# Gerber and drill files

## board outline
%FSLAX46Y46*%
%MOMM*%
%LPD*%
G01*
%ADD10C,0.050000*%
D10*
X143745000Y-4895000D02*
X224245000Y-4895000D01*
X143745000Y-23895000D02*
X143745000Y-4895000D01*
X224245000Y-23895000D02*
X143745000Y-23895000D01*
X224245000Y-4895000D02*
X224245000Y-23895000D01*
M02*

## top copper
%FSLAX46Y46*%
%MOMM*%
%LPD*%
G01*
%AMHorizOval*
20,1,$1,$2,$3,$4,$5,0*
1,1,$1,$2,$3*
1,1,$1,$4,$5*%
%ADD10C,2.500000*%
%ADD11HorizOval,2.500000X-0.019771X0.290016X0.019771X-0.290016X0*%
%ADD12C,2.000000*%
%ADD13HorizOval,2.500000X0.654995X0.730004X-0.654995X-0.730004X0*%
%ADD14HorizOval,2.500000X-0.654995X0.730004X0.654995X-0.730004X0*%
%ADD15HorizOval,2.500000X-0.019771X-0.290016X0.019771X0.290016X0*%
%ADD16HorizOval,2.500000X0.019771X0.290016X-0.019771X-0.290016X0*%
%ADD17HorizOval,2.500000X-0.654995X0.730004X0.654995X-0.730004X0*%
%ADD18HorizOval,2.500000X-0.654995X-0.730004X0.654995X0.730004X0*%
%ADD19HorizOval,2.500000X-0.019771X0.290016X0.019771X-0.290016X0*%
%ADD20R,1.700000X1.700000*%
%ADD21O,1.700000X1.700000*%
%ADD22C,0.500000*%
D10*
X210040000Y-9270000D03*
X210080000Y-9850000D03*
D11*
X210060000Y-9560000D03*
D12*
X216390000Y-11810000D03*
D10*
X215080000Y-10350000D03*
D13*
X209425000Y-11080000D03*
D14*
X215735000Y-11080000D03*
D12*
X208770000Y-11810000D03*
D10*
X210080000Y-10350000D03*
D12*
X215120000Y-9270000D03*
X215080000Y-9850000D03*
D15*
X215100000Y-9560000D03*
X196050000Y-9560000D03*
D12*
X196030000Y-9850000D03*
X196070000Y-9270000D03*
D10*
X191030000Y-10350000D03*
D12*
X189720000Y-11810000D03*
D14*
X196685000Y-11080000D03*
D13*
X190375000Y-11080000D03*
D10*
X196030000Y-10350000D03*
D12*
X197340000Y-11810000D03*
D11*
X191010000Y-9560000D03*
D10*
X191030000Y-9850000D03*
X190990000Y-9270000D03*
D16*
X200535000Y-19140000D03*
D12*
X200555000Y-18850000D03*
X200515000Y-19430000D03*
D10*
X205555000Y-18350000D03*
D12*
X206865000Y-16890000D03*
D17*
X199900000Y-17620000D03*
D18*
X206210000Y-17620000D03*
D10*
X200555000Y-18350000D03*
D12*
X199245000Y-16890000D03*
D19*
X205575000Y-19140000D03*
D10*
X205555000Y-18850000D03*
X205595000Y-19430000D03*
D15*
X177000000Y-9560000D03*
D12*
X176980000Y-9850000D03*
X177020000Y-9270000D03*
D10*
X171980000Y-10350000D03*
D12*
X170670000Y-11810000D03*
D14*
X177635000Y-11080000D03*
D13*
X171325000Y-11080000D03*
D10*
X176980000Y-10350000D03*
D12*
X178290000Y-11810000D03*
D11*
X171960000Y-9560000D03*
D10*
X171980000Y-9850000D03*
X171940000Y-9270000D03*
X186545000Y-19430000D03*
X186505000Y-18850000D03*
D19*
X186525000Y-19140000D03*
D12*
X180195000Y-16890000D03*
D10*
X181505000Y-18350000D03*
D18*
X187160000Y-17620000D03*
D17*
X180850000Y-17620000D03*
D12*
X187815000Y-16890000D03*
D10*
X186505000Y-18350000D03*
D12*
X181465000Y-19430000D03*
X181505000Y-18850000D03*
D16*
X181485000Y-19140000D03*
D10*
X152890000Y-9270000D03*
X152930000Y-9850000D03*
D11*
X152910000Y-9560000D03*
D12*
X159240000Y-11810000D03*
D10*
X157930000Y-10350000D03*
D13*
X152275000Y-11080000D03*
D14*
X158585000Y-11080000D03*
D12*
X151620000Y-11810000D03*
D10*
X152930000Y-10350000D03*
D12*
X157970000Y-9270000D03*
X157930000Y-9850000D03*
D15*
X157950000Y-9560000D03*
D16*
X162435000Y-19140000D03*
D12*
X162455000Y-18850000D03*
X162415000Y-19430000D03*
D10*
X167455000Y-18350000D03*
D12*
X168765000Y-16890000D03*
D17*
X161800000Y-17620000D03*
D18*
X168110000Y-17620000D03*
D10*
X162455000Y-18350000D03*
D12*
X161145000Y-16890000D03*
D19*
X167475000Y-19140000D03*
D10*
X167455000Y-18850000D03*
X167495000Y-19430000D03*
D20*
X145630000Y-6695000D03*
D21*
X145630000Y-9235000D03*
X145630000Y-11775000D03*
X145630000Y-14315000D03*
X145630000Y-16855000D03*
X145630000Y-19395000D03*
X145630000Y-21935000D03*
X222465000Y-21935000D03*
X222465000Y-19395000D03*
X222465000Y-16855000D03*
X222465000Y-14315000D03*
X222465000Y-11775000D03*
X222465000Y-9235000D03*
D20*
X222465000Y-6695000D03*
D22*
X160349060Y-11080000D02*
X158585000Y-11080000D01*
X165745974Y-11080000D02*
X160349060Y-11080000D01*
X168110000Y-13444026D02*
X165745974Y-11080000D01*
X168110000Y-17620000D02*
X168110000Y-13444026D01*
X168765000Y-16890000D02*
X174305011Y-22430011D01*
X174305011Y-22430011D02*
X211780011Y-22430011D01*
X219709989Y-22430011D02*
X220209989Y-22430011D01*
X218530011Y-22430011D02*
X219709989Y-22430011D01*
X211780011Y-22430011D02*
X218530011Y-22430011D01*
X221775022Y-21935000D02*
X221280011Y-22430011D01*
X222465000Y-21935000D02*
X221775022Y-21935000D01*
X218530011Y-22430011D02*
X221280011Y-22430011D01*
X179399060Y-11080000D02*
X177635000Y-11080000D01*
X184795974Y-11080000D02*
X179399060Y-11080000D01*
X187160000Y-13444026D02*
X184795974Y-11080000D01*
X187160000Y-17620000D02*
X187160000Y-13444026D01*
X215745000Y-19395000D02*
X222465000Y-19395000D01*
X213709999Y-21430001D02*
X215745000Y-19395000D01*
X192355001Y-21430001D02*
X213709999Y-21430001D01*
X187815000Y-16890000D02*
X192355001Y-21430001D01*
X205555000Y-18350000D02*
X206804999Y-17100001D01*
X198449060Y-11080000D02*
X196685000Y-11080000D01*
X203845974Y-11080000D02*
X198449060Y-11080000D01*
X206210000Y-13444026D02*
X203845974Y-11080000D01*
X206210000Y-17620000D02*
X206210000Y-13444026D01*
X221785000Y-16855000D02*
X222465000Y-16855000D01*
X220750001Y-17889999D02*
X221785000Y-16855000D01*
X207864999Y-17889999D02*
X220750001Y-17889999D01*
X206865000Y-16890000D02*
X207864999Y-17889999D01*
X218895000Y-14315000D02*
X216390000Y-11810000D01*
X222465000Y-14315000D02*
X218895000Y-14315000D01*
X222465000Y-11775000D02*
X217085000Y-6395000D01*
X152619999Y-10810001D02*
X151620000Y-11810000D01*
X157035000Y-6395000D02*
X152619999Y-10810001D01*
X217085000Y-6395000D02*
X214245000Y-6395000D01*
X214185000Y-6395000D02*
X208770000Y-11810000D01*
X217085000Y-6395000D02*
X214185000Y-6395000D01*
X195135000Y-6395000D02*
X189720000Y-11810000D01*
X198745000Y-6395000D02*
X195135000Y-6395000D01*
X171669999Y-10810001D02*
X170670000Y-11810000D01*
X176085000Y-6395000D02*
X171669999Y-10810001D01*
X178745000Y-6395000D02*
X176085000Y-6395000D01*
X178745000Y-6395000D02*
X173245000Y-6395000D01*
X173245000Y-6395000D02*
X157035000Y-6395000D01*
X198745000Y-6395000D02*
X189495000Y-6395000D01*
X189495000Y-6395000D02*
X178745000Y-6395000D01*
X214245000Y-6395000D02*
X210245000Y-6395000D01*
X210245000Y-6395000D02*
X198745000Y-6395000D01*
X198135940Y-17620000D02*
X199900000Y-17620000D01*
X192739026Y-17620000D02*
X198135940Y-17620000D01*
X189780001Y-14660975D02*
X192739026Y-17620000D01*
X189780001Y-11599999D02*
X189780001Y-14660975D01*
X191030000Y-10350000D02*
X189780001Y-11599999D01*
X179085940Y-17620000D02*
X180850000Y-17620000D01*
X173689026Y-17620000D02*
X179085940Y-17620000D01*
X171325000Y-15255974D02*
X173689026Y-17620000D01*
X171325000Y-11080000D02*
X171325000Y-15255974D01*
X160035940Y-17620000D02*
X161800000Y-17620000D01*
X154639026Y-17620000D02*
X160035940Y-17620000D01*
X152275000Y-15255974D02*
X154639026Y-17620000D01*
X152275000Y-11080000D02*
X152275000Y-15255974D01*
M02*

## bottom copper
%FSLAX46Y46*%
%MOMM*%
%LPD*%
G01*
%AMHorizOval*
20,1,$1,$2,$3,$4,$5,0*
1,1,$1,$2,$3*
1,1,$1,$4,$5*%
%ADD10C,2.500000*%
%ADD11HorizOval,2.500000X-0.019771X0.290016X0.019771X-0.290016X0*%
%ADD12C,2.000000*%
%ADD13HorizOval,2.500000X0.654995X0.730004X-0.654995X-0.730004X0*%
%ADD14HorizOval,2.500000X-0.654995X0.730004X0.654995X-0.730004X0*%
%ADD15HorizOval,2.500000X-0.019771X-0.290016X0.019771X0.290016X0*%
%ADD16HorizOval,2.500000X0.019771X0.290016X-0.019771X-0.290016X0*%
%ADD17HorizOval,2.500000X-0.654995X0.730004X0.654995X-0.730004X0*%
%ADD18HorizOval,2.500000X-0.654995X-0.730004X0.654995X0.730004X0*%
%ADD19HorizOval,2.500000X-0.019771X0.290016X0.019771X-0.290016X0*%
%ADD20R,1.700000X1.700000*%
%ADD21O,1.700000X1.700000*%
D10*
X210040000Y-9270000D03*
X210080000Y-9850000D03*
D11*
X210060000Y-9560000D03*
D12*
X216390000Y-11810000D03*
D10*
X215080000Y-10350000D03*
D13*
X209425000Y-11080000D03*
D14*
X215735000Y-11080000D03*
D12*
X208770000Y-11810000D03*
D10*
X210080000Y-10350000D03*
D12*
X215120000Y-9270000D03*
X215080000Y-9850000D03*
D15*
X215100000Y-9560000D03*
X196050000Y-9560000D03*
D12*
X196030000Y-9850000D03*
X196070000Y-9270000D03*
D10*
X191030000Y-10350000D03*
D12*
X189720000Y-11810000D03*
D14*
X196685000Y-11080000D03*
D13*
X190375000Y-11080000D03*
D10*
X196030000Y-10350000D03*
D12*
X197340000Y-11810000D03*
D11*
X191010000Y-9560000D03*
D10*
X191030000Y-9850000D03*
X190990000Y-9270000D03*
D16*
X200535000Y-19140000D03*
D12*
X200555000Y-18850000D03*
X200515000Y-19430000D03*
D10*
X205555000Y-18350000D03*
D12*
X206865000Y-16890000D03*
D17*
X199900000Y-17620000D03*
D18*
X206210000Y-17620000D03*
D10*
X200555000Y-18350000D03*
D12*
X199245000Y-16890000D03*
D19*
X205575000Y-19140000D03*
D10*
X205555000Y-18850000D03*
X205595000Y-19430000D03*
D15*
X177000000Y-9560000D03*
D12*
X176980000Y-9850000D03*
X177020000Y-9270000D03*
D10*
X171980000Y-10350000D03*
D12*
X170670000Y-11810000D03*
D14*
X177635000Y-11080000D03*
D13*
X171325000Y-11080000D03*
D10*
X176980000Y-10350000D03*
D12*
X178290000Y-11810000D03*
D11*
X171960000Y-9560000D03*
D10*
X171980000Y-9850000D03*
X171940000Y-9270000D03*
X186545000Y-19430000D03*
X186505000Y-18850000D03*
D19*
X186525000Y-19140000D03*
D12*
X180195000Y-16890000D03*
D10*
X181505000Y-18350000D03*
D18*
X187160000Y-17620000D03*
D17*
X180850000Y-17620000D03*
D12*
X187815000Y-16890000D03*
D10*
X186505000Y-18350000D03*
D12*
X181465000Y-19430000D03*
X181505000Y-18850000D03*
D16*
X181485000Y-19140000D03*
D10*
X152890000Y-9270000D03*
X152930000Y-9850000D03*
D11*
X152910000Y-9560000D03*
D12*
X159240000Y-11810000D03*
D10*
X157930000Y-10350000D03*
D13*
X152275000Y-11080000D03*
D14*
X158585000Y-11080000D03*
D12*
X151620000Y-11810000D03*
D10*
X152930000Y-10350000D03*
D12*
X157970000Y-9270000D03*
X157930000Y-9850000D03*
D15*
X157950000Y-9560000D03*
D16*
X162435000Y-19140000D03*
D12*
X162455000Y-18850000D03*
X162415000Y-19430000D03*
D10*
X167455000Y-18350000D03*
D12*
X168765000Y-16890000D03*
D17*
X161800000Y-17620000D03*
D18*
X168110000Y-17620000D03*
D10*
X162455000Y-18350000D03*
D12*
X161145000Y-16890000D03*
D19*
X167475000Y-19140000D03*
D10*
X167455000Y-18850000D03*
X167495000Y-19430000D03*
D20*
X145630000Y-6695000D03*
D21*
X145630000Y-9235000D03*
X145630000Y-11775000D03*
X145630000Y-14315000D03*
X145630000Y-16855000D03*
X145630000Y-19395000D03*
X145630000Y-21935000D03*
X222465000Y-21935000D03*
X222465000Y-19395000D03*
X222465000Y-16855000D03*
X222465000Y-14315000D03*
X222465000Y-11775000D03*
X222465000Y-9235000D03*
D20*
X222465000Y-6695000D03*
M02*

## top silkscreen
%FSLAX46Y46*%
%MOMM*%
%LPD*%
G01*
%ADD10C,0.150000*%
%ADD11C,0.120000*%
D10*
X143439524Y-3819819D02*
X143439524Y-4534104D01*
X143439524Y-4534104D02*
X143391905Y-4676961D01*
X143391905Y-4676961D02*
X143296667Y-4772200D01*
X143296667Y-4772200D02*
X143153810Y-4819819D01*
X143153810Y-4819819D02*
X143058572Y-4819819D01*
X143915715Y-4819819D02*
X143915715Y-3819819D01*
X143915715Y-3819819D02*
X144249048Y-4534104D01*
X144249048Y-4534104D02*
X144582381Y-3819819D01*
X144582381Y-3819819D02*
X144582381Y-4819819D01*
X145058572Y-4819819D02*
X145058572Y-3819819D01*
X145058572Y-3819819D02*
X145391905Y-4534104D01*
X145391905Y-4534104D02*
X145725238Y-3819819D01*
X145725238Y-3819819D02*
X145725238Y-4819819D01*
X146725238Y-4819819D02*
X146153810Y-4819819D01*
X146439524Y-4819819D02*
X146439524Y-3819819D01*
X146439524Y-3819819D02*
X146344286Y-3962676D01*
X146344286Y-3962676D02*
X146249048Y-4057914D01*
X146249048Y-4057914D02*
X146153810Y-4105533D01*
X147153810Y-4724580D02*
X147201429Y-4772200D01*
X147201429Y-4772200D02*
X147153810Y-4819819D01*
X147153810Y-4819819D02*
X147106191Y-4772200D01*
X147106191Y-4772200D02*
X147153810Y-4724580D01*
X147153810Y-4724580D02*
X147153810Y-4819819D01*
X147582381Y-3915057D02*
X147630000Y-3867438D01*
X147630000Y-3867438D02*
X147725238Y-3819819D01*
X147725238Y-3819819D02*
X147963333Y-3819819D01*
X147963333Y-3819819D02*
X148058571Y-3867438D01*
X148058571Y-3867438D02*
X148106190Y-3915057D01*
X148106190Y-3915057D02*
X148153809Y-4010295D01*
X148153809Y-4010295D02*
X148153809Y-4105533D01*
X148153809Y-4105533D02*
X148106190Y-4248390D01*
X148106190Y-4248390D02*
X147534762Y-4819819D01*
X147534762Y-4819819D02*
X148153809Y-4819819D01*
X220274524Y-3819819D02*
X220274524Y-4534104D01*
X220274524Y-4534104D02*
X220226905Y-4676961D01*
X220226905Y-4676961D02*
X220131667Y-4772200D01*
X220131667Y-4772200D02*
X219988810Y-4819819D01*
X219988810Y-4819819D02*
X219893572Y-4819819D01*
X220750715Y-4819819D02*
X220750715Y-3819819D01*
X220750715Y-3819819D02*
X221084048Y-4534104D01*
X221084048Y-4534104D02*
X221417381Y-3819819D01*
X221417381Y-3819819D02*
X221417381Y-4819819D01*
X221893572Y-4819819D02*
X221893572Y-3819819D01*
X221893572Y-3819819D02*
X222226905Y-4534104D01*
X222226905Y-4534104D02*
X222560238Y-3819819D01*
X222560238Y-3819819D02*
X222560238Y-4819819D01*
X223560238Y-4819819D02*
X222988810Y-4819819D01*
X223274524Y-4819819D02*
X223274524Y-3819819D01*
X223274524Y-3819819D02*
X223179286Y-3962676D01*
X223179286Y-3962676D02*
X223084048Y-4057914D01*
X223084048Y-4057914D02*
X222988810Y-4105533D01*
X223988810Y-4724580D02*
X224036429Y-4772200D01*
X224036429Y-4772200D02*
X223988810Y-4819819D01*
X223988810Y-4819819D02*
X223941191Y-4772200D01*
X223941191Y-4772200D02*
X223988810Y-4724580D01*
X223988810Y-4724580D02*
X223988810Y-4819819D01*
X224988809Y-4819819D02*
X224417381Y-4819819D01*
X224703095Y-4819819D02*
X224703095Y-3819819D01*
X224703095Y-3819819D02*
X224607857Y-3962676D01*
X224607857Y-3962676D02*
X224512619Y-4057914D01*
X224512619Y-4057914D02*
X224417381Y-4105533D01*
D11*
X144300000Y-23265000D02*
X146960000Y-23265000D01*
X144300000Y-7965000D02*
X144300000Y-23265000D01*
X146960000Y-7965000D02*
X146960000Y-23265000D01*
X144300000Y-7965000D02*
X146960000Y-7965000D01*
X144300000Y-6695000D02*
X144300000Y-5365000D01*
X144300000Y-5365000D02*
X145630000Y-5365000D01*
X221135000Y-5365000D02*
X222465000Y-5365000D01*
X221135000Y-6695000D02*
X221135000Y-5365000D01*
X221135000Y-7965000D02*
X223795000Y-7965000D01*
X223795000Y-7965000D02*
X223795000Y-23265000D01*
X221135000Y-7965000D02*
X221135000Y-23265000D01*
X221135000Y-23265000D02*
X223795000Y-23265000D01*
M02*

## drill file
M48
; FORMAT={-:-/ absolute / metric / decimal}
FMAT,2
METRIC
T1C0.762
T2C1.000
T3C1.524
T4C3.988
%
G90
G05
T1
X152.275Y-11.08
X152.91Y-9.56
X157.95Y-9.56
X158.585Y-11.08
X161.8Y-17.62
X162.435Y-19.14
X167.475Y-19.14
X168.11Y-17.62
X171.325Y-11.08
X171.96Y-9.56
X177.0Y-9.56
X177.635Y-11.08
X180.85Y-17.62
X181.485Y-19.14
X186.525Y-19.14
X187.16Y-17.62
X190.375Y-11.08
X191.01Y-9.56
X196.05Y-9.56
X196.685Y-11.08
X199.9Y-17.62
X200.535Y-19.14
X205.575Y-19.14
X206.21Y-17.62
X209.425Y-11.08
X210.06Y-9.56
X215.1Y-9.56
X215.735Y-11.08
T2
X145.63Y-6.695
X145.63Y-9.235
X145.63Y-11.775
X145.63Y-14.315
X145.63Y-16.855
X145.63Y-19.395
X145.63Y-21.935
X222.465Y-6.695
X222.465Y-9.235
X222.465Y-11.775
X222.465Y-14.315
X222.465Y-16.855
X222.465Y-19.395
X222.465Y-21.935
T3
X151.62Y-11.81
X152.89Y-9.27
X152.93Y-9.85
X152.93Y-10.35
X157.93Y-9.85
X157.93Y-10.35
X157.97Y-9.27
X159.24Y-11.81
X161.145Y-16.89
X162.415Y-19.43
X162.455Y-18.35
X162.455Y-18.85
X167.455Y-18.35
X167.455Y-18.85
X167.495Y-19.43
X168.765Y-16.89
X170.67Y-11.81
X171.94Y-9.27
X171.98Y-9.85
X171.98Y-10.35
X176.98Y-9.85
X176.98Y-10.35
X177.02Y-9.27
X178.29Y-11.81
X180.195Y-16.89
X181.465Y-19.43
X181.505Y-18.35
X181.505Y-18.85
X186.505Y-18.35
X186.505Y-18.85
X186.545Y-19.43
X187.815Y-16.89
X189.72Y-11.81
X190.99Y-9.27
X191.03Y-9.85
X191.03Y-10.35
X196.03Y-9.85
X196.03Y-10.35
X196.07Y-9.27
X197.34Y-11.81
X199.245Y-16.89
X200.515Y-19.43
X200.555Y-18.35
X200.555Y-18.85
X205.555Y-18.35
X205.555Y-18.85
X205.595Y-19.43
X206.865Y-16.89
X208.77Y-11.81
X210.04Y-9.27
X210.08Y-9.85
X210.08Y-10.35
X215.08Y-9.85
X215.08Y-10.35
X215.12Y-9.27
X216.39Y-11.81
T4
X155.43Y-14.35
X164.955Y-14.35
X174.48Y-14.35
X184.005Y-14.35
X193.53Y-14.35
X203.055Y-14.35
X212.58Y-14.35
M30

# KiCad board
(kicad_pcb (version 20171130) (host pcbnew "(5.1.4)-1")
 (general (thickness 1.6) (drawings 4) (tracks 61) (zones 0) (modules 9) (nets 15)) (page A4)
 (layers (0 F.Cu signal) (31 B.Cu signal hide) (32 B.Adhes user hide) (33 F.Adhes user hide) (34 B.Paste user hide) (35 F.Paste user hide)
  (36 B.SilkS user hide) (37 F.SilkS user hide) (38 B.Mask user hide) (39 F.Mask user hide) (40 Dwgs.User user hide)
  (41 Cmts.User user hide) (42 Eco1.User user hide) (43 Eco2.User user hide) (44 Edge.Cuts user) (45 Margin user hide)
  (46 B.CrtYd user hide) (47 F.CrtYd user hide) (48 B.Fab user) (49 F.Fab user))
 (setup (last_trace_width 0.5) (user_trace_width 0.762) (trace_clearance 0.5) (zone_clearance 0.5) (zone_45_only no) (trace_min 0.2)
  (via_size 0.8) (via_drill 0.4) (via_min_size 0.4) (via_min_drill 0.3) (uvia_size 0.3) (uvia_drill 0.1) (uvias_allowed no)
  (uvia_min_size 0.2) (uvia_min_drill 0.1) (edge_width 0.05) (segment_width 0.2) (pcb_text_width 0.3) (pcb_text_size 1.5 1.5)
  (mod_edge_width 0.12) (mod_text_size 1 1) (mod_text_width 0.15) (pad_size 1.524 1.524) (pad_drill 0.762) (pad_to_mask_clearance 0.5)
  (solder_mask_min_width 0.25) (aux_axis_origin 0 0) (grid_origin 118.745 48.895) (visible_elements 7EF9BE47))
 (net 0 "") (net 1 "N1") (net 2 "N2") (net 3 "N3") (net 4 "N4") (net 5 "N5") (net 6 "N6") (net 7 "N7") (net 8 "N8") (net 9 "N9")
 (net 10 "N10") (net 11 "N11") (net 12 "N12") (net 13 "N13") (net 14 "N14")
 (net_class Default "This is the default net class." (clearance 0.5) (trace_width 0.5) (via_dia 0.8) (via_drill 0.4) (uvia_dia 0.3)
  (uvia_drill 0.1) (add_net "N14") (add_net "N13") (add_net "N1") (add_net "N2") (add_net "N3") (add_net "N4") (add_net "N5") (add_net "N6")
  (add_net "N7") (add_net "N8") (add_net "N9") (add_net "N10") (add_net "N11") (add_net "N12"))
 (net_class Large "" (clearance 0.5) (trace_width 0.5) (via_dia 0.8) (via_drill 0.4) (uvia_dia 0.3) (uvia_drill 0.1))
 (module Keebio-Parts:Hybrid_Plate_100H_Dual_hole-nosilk (layer F.Cu) (at 212.58 14.35)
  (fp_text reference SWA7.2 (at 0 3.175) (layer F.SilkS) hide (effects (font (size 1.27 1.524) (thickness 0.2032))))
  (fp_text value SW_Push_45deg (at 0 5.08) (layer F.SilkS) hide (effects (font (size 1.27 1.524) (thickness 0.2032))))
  (pad 1 thru_hole circle (at -2.54 -5.08 330.9) (size 2.5 2.5) (drill 1.524) (layers *.Cu F.Mask) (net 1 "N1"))
  (pad 1 thru_hole circle (at -2.5 -4.5 330.9) (size 2.5 2.5) (drill 1.524) (layers *.Cu F.Mask) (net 1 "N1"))
  (pad 1 thru_hole oval (at -2.52 -4.79 3.9) (size 2.5 3.081378) (drill 0.762) (layers *.Cu F.Mask) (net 1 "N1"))
  (pad 2 thru_hole circle (at 3.81 -2.54 330.9) (size 2 2) (drill 1.524) (layers *.Cu F.Mask) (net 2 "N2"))
  (pad 2 thru_hole circle (at 2.5 -4) (size 2.5 2.5) (drill 1.524) (layers *.Cu *.Mask) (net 2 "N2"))
  (pad 1 thru_hole oval (at -3.155 -3.27 138.1) (size 2.5 4.461556) (drill 0.762) (layers *.Cu B.Mask) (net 1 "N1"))
  (pad 2 thru_hole oval (at 3.155 -3.27 221.9) (size 2.5 4.461556) (drill 0.762) (layers *.Cu F.Mask) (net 2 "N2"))
  (pad 1 thru_hole circle (at -3.81 -2.54 330.9) (size 2 2) (drill 1.524) (layers *.Cu B.Mask) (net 1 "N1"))
  (pad HOLE np_thru_hole circle (at 0 0) (size 3.9878 3.9878) (drill 3.9878) (layers *.Cu *.Mask))
  (pad 1 thru_hole circle (at -2.5 -4 330.9) (size 2.5 2.5) (drill 1.524) (layers *.Cu *.Mask) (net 1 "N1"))
  (pad 2 thru_hole circle (at 2.54 -5.08 330.9) (size 2 2) (drill 1.524) (layers *.Cu B.Mask) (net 2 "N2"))
  (pad 2 thru_hole circle (at 2.5 -4.5 330.9) (size 2 2) (drill 1.524) (layers *.Cu B.Mask) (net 2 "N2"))
  (pad 2 thru_hole oval (at 2.52 -4.79 356.1) (size 2.5 3.081378) (drill 0.762) (layers *.Cu B.Mask) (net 2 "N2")))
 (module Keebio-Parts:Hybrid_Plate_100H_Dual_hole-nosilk (layer F.Cu) (at 193.53 14.35)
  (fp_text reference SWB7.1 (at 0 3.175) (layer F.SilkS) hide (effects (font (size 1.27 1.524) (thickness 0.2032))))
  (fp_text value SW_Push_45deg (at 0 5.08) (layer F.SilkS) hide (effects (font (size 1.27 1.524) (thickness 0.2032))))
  (pad 2 thru_hole oval (at 2.52 -4.79 356.1) (size 2.5 3.081378) (drill 0.762) (layers *.Cu B.Mask) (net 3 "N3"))
  (pad 2 thru_hole circle (at 2.5 -4.5 330.9) (size 2 2) (drill 1.524) (layers *.Cu B.Mask) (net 3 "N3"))
  (pad 2 thru_hole circle (at 2.54 -5.08 330.9) (size 2 2) (drill 1.524) (layers *.Cu B.Mask) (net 3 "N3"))
  (pad 1 thru_hole circle (at -2.5 -4 330.9) (size 2.5 2.5) (drill 1.524) (layers *.Cu *.Mask) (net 1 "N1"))
  (pad HOLE np_thru_hole circle (at 0 0) (size 3.9878 3.9878) (drill 3.9878) (layers *.Cu *.Mask))
  (pad 1 thru_hole circle (at -3.81 -2.54 330.9) (size 2 2) (drill 1.524) (layers *.Cu B.Mask) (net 1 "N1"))
  (pad 2 thru_hole oval (at 3.155 -3.27 221.9) (size 2.5 4.461556) (drill 0.762) (layers *.Cu F.Mask) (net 3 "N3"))
  (pad 1 thru_hole oval (at -3.155 -3.27 138.1) (size 2.5 4.461556) (drill 0.762) (layers *.Cu B.Mask) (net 1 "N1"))
  (pad 2 thru_hole circle (at 2.5 -4) (size 2.5 2.5) (drill 1.524) (layers *.Cu *.Mask) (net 3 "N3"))
  (pad 2 thru_hole circle (at 3.81 -2.54 330.9) (size 2 2) (drill 1.524) (layers *.Cu F.Mask) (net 3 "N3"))
  (pad 1 thru_hole oval (at -2.52 -4.79 3.9) (size 2.5 3.081378) (drill 0.762) (layers *.Cu F.Mask) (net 1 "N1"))
  (pad 1 thru_hole circle (at -2.5 -4.5 330.9) (size 2.5 2.5) (drill 1.524) (layers *.Cu F.Mask) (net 1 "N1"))
  (pad 1 thru_hole circle (at -2.54 -5.08 330.9) (size 2.5 2.5) (drill 1.524) (layers *.Cu F.Mask) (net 1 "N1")))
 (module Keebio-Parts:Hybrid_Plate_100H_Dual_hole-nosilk (layer F.Cu) (at 203.055 14.35 180)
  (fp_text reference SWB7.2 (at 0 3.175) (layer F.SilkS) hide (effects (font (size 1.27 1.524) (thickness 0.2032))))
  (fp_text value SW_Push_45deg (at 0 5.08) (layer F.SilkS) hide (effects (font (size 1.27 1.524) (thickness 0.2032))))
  (pad 2 thru_hole oval (at 2.52 -4.79 176.1) (size 2.5 3.081378) (drill 0.762) (layers *.Cu B.Mask) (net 1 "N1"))
  (pad 2 thru_hole circle (at 2.5 -4.5 150.9) (size 2 2) (drill 1.524) (layers *.Cu B.Mask) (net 1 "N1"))
  (pad 2 thru_hole circle (at 2.54 -5.08 150.9) (size 2 2) (drill 1.524) (layers *.Cu B.Mask) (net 1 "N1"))
  (pad 1 thru_hole circle (at -2.5 -4 150.9) (size 2.5 2.5) (drill 1.524) (layers *.Cu *.Mask) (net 3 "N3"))
  (pad HOLE np_thru_hole circle (at 0 0 180) (size 3.9878 3.9878) (drill 3.9878) (layers *.Cu *.Mask))
  (pad 1 thru_hole circle (at -3.81 -2.54 150.9) (size 2 2) (drill 1.524) (layers *.Cu B.Mask) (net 3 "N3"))
  (pad 2 thru_hole oval (at 3.155 -3.27 41.9) (size 2.5 4.461556) (drill 0.762) (layers *.Cu F.Mask) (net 1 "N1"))
  (pad 1 thru_hole oval (at -3.155 -3.27 318.1) (size 2.5 4.461556) (drill 0.762) (layers *.Cu B.Mask) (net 3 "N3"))
  (pad 2 thru_hole circle (at 2.5 -4 180) (size 2.5 2.5) (drill 1.524) (layers *.Cu *.Mask) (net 1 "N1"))
  (pad 2 thru_hole circle (at 3.81 -2.54 150.9) (size 2 2) (drill 1.524) (layers *.Cu F.Mask) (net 1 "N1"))
  (pad 1 thru_hole oval (at -2.52 -4.79 183.9) (size 2.5 3.081378) (drill 0.762) (layers *.Cu F.Mask) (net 3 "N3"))
  (pad 1 thru_hole circle (at -2.5 -4.5 150.9) (size 2.5 2.5) (drill 1.524) (layers *.Cu F.Mask) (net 3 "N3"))
  (pad 1 thru_hole circle (at -2.54 -5.08 150.9) (size 2.5 2.5) (drill 1.524) (layers *.Cu F.Mask) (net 3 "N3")))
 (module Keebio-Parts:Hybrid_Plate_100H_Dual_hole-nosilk (layer F.Cu) (at 174.48 14.35)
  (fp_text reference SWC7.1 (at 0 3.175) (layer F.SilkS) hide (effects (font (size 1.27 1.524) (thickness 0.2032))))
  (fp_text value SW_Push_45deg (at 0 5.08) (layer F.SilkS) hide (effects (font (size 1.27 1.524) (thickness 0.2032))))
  (pad 2 thru_hole oval (at 2.52 -4.79 356.1) (size 2.5 3.081378) (drill 0.762) (layers *.Cu B.Mask) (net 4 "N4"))
  (pad 2 thru_hole circle (at 2.5 -4.5 330.9) (size 2 2) (drill 1.524) (layers *.Cu B.Mask) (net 4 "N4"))
  (pad 2 thru_hole circle (at 2.54 -5.08 330.9) (size 2 2) (drill 1.524) (layers *.Cu B.Mask) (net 4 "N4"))
  (pad 1 thru_hole circle (at -2.5 -4 330.9) (size 2.5 2.5) (drill 1.524) (layers *.Cu *.Mask) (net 1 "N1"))
  (pad HOLE np_thru_hole circle (at 0 0) (size 3.9878 3.9878) (drill 3.9878) (layers *.Cu *.Mask))
  (pad 1 thru_hole circle (at -3.81 -2.54 330.9) (size 2 2) (drill 1.524) (layers *.Cu B.Mask) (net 1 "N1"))
  (pad 2 thru_hole oval (at 3.155 -3.27 221.9) (size 2.5 4.461556) (drill 0.762) (layers *.Cu F.Mask) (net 4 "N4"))
  (pad 1 thru_hole oval (at -3.155 -3.27 138.1) (size 2.5 4.461556) (drill 0.762) (layers *.Cu B.Mask) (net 1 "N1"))
  (pad 2 thru_hole circle (at 2.5 -4) (size 2.5 2.5) (drill 1.524) (layers *.Cu *.Mask) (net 4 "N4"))
  (pad 2 thru_hole circle (at 3.81 -2.54 330.9) (size 2 2) (drill 1.524) (layers *.Cu F.Mask) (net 4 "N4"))
  (pad 1 thru_hole oval (at -2.52 -4.79 3.9) (size 2.5 3.081378) (drill 0.762) (layers *.Cu F.Mask) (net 1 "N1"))
  (pad 1 thru_hole circle (at -2.5 -4.5 330.9) (size 2.5 2.5) (drill 1.524) (layers *.Cu F.Mask) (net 1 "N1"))
  (pad 1 thru_hole circle (at -2.54 -5.08 330.9) (size 2.5 2.5) (drill 1.524) (layers *.Cu F.Mask) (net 1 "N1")))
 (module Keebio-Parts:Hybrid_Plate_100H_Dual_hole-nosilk (layer F.Cu) (at 184.005 14.35 180)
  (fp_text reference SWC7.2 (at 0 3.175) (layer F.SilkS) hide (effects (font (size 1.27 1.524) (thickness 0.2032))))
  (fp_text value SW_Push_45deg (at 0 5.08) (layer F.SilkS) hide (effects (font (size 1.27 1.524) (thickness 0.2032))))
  (pad 1 thru_hole circle (at -2.54 -5.08 150.9) (size 2.5 2.5) (drill 1.524) (layers *.Cu F.Mask) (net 4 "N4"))
  (pad 1 thru_hole circle (at -2.5 -4.5 150.9) (size 2.5 2.5) (drill 1.524) (layers *.Cu F.Mask) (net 4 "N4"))
  (pad 1 thru_hole oval (at -2.52 -4.79 183.9) (size 2.5 3.081378) (drill 0.762) (layers *.Cu F.Mask) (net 4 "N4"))
  (pad 2 thru_hole circle (at 3.81 -2.54 150.9) (size 2 2) (drill 1.524) (layers *.Cu F.Mask) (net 1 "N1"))
  (pad 2 thru_hole circle (at 2.5 -4 180) (size 2.5 2.5) (drill 1.524) (layers *.Cu *.Mask) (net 1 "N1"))
  (pad 1 thru_hole oval (at -3.155 -3.27 318.1) (size 2.5 4.461556) (drill 0.762) (layers *.Cu B.Mask) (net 4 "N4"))
  (pad 2 thru_hole oval (at 3.155 -3.27 41.9) (size 2.5 4.461556) (drill 0.762) (layers *.Cu F.Mask) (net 1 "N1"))
  (pad 1 thru_hole circle (at -3.81 -2.54 150.9) (size 2 2) (drill 1.524) (layers *.Cu B.Mask) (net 4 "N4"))
  (pad HOLE np_thru_hole circle (at 0 0 180) (size 3.9878 3.9878) (drill 3.9878) (layers *.Cu *.Mask))
  (pad 1 thru_hole circle (at -2.5 -4 150.9) (size 2.5 2.5) (drill 1.524) (layers *.Cu *.Mask) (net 4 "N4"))
  (pad 2 thru_hole circle (at 2.54 -5.08 150.9) (size 2 2) (drill 1.524) (layers *.Cu B.Mask) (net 1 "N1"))
  (pad 2 thru_hole circle (at 2.5 -4.5 150.9) (size 2 2) (drill 1.524) (layers *.Cu B.Mask) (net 1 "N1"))
  (pad 2 thru_hole oval (at 2.52 -4.79 176.1) (size 2.5 3.081378) (drill 0.762) (layers *.Cu B.Mask) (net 1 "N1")))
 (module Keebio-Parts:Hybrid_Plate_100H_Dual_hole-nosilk (layer F.Cu) (at 155.43 14.35)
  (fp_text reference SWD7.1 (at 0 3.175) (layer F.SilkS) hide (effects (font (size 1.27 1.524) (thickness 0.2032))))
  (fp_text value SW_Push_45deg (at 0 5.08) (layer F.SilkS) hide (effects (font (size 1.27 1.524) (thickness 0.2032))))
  (pad 1 thru_hole circle (at -2.54 -5.08 330.9) (size 2.5 2.5) (drill 1.524) (layers *.Cu F.Mask) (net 1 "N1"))
  (pad 1 thru_hole circle (at -2.5 -4.5 330.9) (size 2.5 2.5) (drill 1.524) (layers *.Cu F.Mask) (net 1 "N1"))
  (pad 1 thru_hole oval (at -2.52 -4.79 3.9) (size 2.5 3.081378) (drill 0.762) (layers *.Cu F.Mask) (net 1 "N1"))
  (pad 2 thru_hole circle (at 3.81 -2.54 330.9) (size 2 2) (drill 1.524) (layers *.Cu F.Mask) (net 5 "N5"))
  (pad 2 thru_hole circle (at 2.5 -4) (size 2.5 2.5) (drill 1.524) (layers *.Cu *.Mask) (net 5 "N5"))
  (pad 1 thru_hole oval (at -3.155 -3.27 138.1) (size 2.5 4.461556) (drill 0.762) (layers *.Cu B.Mask) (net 1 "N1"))
  (pad 2 thru_hole oval (at 3.155 -3.27 221.9) (size 2.5 4.461556) (drill 0.762) (layers *.Cu F.Mask) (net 5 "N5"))
  (pad 1 thru_hole circle (at -3.81 -2.54 330.9) (size 2 2) (drill 1.524) (layers *.Cu B.Mask) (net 1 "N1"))
  (pad HOLE np_thru_hole circle (at 0 0) (size 3.9878 3.9878) (drill 3.9878) (layers *.Cu *.Mask))
  (pad 1 thru_hole circle (at -2.5 -4 330.9) (size 2.5 2.5) (drill 1.524) (layers *.Cu *.Mask) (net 1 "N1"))
  (pad 2 thru_hole circle (at 2.54 -5.08 330.9) (size 2 2) (drill 1.524) (layers *.Cu B.Mask) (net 5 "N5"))
  (pad 2 thru_hole circle (at 2.5 -4.5 330.9) (size 2 2) (drill 1.524) (layers *.Cu B.Mask) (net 5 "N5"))
  (pad 2 thru_hole oval (at 2.52 -4.79 356.1) (size 2.5 3.081378) (drill 0.762) (layers *.Cu B.Mask) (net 5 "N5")))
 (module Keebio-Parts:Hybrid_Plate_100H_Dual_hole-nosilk (layer F.Cu) (at 164.955 14.35 180)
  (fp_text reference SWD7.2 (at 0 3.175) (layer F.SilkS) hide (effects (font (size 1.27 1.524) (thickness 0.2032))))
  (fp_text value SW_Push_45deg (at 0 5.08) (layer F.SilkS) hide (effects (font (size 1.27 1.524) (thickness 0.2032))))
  (pad 2 thru_hole oval (at 2.52 -4.79 176.1) (size 2.5 3.081378) (drill 0.762) (layers *.Cu B.Mask) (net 1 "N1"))
  (pad 2 thru_hole circle (at 2.5 -4.5 150.9) (size 2 2) (drill 1.524) (layers *.Cu B.Mask) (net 1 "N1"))
  (pad 2 thru_hole circle (at 2.54 -5.08 150.9) (size 2 2) (drill 1.524) (layers *.Cu B.Mask) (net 1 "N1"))
  (pad 1 thru_hole circle (at -2.5 -4 150.9) (size 2.5 2.5) (drill 1.524) (layers *.Cu *.Mask) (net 5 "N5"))
  (pad HOLE np_thru_hole circle (at 0 0 180) (size 3.9878 3.9878) (drill 3.9878) (layers *.Cu *.Mask))
  (pad 1 thru_hole circle (at -3.81 -2.54 150.9) (size 2 2) (drill 1.524) (layers *.Cu B.Mask) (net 5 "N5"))
  (pad 2 thru_hole oval (at 3.155 -3.27 41.9) (size 2.5 4.461556) (drill 0.762) (layers *.Cu F.Mask) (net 1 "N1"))
  (pad 1 thru_hole oval (at -3.155 -3.27 318.1) (size 2.5 4.461556) (drill 0.762) (layers *.Cu B.Mask) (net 5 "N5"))
  (pad 2 thru_hole circle (at 2.5 -4 180) (size 2.5 2.5) (drill 1.524) (layers *.Cu *.Mask) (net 1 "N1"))
  (pad 2 thru_hole circle (at 3.81 -2.54 150.9) (size 2 2) (drill 1.524) (layers *.Cu F.Mask) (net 1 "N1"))
  (pad 1 thru_hole oval (at -2.52 -4.79 183.9) (size 2.5 3.081378) (drill 0.762) (layers *.Cu F.Mask) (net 5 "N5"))
  (pad 1 thru_hole circle (at -2.5 -4.5 150.9) (size 2.5 2.5) (drill 1.524) (layers *.Cu F.Mask) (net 5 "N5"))
  (pad 1 thru_hole circle (at -2.54 -5.08 150.9) (size 2.5 2.5) (drill 1.524) (layers *.Cu F.Mask) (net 5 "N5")))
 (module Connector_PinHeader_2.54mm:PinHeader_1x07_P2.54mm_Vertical (layer F.Cu) (at 145.63 6.695)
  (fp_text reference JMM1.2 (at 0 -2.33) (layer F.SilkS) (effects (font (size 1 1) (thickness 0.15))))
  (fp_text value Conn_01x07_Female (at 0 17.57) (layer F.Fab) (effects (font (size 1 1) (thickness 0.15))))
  (fp_line (start -1.33 16.57) (end 1.33 16.57) (layer F.SilkS) (width 0.12))
  (fp_line (start -1.33 1.27) (end -1.33 16.57) (layer F.SilkS) (width 0.12))
  (fp_line (start 1.33 1.27) (end 1.33 16.57) (layer F.SilkS) (width 0.12))
  (fp_line (start -1.33 1.27) (end 1.33 1.27) (layer F.SilkS) (width 0.12))
  (fp_line (start -1.33 0) (end -1.33 -1.33) (layer F.SilkS) (width 0.12))
  (fp_line (start -1.33 -1.33) (end 0 -1.33) (layer F.SilkS) (width 0.12))
  (pad 1 thru_hole rect (at 0 0) (size 1.7 1.7) (drill 1) (layers *.Cu *.Mask) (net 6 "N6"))
  (pad 2 thru_hole oval (at 0 2.54) (size 1.7 1.7) (drill 1) (layers *.Cu *.Mask) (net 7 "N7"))
  (pad 3 thru_hole oval (at 0 5.08) (size 1.7 1.7) (drill 1) (layers *.Cu *.Mask) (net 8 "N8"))
  (pad 4 thru_hole oval (at 0 7.62) (size 1.7 1.7) (drill 1) (layers *.Cu *.Mask) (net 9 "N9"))
  (pad 5 thru_hole oval (at 0 10.16) (size 1.7 1.7) (drill 1) (layers *.Cu *.Mask) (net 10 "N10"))
  (pad 6 thru_hole oval (at 0 12.7) (size 1.7 1.7) (drill 1) (layers *.Cu *.Mask) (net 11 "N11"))
  (pad 7 thru_hole oval (at 0 15.24) (size 1.7 1.7) (drill 1) (layers *.Cu *.Mask) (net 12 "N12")))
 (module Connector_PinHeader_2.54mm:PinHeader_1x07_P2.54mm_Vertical (layer F.Cu) (at 222.465 6.695)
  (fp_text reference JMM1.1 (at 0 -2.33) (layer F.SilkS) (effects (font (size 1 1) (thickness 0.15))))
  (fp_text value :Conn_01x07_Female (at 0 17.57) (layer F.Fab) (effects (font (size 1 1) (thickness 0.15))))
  (fp_line (start -1.33 -1.33) (end 0 -1.33) (layer F.SilkS) (width 0.12))
  (fp_line (start -1.33 0) (end -1.33 -1.33) (layer F.SilkS) (width 0.12))
  (fp_line (start -1.33 1.27) (end 1.33 1.27) (layer F.SilkS) (width 0.12))
  (fp_line (start 1.33 1.27) (end 1.33 16.57) (layer F.SilkS) (width 0.12))
  (fp_line (start -1.33 1.27) (end -1.33 16.57) (layer F.SilkS) (width 0.12))
  (fp_line (start -1.33 16.57) (end 1.33 16.57) (layer F.SilkS) (width 0.12))
  (pad 7 thru_hole oval (at 0 15.24) (size 1.7 1.7) (drill 1) (layers *.Cu *.Mask) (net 5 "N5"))
  (pad 6 thru_hole oval (at 0 12.7) (size 1.7 1.7) (drill 1) (layers *.Cu *.Mask) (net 4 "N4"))
  (pad 5 thru_hole oval (at 0 10.16) (size 1.7 1.7) (drill 1) (layers *.Cu *.Mask) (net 3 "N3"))
  (pad 4 thru_hole oval (at 0 7.62) (size 1.7 1.7) (drill 1) (layers *.Cu *.Mask) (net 2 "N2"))
  (pad 3 thru_hole oval (at 0 5.08) (size 1.7 1.7) (drill 1) (layers *.Cu *.Mask) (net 1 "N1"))
  (pad 2 thru_hole oval (at 0 2.54) (size 1.7 1.7) (drill 1) (layers *.Cu *.Mask) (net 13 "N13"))
  (pad 1 thru_hole rect (at 0 0) (size 1.7 1.7) (drill 1) (layers *.Cu *.Mask) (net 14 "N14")))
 (gr_line (start 143.745 4.895) (end 224.245 4.895) (layer Edge.Cuts) (width 0.05))
 (gr_line (start 143.745 23.895) (end 143.745 4.895) (layer Edge.Cuts) (width 0.05))
 (gr_line (start 224.245 23.895) (end 143.745 23.895) (layer Edge.Cuts) (width 0.05))
 (gr_line (start 224.245 4.895) (end 224.245 23.895) (layer Edge.Cuts) (width 0.05))
 (segment (start 160.34906 11.08) (end 158.585 11.08) (width 0.5) (layer F.Cu) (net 5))
 (segment (start 165.745974 11.08) (end 160.34906 11.08) (width 0.5) (layer F.Cu) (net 5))
 (segment (start 168.11 13.444026) (end 165.745974 11.08) (width 0.5) (layer F.Cu) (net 5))
 (segment (start 168.11 17.62) (end 168.11 13.444026) (width 0.5) (layer F.Cu) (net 5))
 (segment (start 168.765 16.89) (end 174.305011 22.430011) (width 0.5) (layer F.Cu) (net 5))
 (segment (start 174.305011 22.430011) (end 211.780011 22.430011) (width 0.5) (layer F.Cu) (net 5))
 (segment (start 219.709989 22.430011) (end 220.209989 22.430011) (width 0.5) (layer F.Cu) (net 5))
 (segment (start 218.530011 22.430011) (end 219.709989 22.430011) (width 0.5) (layer F.Cu) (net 5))
 (segment (start 211.780011 22.430011) (end 218.530011 22.430011) (width 0.5) (layer F.Cu) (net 5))
 (segment (start 221.775022 21.935) (end 221.280011 22.430011) (width 0.5) (layer F.Cu) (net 5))
 (segment (start 222.465 21.935) (end 221.775022 21.935) (width 0.5) (layer F.Cu) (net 5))
 (segment (start 218.530011 22.430011) (end 221.280011 22.430011) (width 0.5) (layer F.Cu) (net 5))
 (segment (start 179.39906 11.08) (end 177.635 11.08) (width 0.5) (layer F.Cu) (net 4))
 (segment (start 184.795974 11.08) (end 179.39906 11.08) (width 0.5) (layer F.Cu) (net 4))
 (segment (start 187.16 13.444026) (end 184.795974 11.08) (width 0.5) (layer F.Cu) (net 4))
 (segment (start 187.16 17.62) (end 187.16 13.444026) (width 0.5) (layer F.Cu) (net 4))
 (segment (start 215.745 19.395) (end 222.465 19.395) (width 0.5) (layer F.Cu) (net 4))
 (segment (start 213.709999 21.430001) (end 215.745 19.395) (width 0.5) (layer F.Cu) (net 4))
 (segment (start 192.355001 21.430001) (end 213.709999 21.430001) (width 0.5) (layer F.Cu) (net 4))
 (segment (start 187.815 16.89) (end 192.355001 21.430001) (width 0.5) (layer F.Cu) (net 4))
 (segment (start 205.555 18.35) (end 206.804999 17.100001) (width 0.5) (layer F.Cu) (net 3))
 (segment (start 198.44906 11.08) (end 196.685 11.08) (width 0.5) (layer F.Cu) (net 3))
 (segment (start 203.845974 11.08) (end 198.44906 11.08) (width 0.5) (layer F.Cu) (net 3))
 (segment (start 206.21 13.444026) (end 203.845974 11.08) (width 0.5) (layer F.Cu) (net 3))
 (segment (start 206.21 17.62) (end 206.21 13.444026) (width 0.5) (layer F.Cu) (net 3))
 (segment (start 221.785 16.855) (end 222.465 16.855) (width 0.5) (layer F.Cu) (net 3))
 (segment (start 220.750001 17.889999) (end 221.785 16.855) (width 0.5) (layer F.Cu) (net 3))
 (segment (start 207.864999 17.889999) (end 220.750001 17.889999) (width 0.5) (layer F.Cu) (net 3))
 (segment (start 206.865 16.89) (end 207.864999 17.889999) (width 0.5) (layer F.Cu) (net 3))
 (segment (start 218.895 14.315) (end 216.39 11.81) (width 0.5) (layer F.Cu) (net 2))
 (segment (start 222.465 14.315) (end 218.895 14.315) (width 0.5) (layer F.Cu) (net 2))
 (segment (start 222.465 11.775) (end 217.085 6.395) (width 0.5) (layer F.Cu) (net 1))
 (segment (start 152.619999 10.810001) (end 151.62 11.81) (width 0.5) (layer F.Cu) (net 1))
 (segment (start 157.035 6.395) (end 152.619999 10.810001) (width 0.5) (layer F.Cu) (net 1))
 (segment (start 217.085 6.395) (end 214.245 6.395) (width 0.5) (layer F.Cu) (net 1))
 (segment (start 214.185 6.395) (end 208.77 11.81) (width 0.5) (layer F.Cu) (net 1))
 (segment (start 217.085 6.395) (end 214.185 6.395) (width 0.5) (layer F.Cu) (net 1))
 (segment (start 195.135 6.395) (end 189.72 11.81) (width 0.5) (layer F.Cu) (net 1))
 (segment (start 198.745 6.395) (end 195.135 6.395) (width 0.5) (layer F.Cu) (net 1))
 (segment (start 171.669999 10.810001) (end 170.67 11.81) (width 0.5) (layer F.Cu) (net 1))
 (segment (start 176.085 6.395) (end 171.669999 10.810001) (width 0.5) (layer F.Cu) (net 1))
 (segment (start 178.745 6.395) (end 176.085 6.395) (width 0.5) (layer F.Cu) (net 1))
 (segment (start 178.745 6.395) (end 173.245 6.395) (width 0.5) (layer F.Cu) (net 1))
 (segment (start 173.245 6.395) (end 157.035 6.395) (width 0.5) (layer F.Cu) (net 1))
 (segment (start 198.745 6.395) (end 189.495 6.395) (width 0.5) (layer F.Cu) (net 1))
 (segment (start 189.495 6.395) (end 178.745 6.395) (width 0.5) (layer F.Cu) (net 1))
 (segment (start 214.245 6.395) (end 210.245 6.395) (width 0.5) (layer F.Cu) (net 1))
 (segment (start 210.245 6.395) (end 198.745 6.395) (width 0.5) (layer F.Cu) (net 1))
 (segment (start 198.13594 17.62) (end 199.9 17.62) (width 0.5) (layer F.Cu) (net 1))
 (segment (start 192.739026 17.62) (end 198.13594 17.62) (width 0.5) (layer F.Cu) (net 1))
 (segment (start 189.780001 14.660975) (end 192.739026 17.62) (width 0.5) (layer F.Cu) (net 1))
 (segment (start 189.780001 11.599999) (end 189.780001 14.660975) (width 0.5) (layer F.Cu) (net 1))
 (segment (start 191.03 10.35) (end 189.780001 11.599999) (width 0.5) (layer F.Cu) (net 1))
 (segment (start 179.08594 17.62) (end 180.85 17.62) (width 0.5) (layer F.Cu) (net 1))
 (segment (start 173.689026 17.62) (end 179.08594 17.62) (width 0.5) (layer F.Cu) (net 1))
 (segment (start 171.325 15.255974) (end 173.689026 17.62) (width 0.5) (layer F.Cu) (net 1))
 (segment (start 171.325 11.08) (end 171.325 15.255974) (width 0.5) (layer F.Cu) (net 1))
 (segment (start 160.03594 17.62) (end 161.8 17.62) (width 0.5) (layer F.Cu) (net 1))
 (segment (start 154.639026 17.62) (end 160.03594 17.62) (width 0.5) (layer F.Cu) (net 1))
 (segment (start 152.275 15.255974) (end 154.639026 17.62) (width 0.5) (layer F.Cu) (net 1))
 (segment (start 152.275 11.08) (end 152.275 15.255974) (width 0.5) (layer F.Cu) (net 1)))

